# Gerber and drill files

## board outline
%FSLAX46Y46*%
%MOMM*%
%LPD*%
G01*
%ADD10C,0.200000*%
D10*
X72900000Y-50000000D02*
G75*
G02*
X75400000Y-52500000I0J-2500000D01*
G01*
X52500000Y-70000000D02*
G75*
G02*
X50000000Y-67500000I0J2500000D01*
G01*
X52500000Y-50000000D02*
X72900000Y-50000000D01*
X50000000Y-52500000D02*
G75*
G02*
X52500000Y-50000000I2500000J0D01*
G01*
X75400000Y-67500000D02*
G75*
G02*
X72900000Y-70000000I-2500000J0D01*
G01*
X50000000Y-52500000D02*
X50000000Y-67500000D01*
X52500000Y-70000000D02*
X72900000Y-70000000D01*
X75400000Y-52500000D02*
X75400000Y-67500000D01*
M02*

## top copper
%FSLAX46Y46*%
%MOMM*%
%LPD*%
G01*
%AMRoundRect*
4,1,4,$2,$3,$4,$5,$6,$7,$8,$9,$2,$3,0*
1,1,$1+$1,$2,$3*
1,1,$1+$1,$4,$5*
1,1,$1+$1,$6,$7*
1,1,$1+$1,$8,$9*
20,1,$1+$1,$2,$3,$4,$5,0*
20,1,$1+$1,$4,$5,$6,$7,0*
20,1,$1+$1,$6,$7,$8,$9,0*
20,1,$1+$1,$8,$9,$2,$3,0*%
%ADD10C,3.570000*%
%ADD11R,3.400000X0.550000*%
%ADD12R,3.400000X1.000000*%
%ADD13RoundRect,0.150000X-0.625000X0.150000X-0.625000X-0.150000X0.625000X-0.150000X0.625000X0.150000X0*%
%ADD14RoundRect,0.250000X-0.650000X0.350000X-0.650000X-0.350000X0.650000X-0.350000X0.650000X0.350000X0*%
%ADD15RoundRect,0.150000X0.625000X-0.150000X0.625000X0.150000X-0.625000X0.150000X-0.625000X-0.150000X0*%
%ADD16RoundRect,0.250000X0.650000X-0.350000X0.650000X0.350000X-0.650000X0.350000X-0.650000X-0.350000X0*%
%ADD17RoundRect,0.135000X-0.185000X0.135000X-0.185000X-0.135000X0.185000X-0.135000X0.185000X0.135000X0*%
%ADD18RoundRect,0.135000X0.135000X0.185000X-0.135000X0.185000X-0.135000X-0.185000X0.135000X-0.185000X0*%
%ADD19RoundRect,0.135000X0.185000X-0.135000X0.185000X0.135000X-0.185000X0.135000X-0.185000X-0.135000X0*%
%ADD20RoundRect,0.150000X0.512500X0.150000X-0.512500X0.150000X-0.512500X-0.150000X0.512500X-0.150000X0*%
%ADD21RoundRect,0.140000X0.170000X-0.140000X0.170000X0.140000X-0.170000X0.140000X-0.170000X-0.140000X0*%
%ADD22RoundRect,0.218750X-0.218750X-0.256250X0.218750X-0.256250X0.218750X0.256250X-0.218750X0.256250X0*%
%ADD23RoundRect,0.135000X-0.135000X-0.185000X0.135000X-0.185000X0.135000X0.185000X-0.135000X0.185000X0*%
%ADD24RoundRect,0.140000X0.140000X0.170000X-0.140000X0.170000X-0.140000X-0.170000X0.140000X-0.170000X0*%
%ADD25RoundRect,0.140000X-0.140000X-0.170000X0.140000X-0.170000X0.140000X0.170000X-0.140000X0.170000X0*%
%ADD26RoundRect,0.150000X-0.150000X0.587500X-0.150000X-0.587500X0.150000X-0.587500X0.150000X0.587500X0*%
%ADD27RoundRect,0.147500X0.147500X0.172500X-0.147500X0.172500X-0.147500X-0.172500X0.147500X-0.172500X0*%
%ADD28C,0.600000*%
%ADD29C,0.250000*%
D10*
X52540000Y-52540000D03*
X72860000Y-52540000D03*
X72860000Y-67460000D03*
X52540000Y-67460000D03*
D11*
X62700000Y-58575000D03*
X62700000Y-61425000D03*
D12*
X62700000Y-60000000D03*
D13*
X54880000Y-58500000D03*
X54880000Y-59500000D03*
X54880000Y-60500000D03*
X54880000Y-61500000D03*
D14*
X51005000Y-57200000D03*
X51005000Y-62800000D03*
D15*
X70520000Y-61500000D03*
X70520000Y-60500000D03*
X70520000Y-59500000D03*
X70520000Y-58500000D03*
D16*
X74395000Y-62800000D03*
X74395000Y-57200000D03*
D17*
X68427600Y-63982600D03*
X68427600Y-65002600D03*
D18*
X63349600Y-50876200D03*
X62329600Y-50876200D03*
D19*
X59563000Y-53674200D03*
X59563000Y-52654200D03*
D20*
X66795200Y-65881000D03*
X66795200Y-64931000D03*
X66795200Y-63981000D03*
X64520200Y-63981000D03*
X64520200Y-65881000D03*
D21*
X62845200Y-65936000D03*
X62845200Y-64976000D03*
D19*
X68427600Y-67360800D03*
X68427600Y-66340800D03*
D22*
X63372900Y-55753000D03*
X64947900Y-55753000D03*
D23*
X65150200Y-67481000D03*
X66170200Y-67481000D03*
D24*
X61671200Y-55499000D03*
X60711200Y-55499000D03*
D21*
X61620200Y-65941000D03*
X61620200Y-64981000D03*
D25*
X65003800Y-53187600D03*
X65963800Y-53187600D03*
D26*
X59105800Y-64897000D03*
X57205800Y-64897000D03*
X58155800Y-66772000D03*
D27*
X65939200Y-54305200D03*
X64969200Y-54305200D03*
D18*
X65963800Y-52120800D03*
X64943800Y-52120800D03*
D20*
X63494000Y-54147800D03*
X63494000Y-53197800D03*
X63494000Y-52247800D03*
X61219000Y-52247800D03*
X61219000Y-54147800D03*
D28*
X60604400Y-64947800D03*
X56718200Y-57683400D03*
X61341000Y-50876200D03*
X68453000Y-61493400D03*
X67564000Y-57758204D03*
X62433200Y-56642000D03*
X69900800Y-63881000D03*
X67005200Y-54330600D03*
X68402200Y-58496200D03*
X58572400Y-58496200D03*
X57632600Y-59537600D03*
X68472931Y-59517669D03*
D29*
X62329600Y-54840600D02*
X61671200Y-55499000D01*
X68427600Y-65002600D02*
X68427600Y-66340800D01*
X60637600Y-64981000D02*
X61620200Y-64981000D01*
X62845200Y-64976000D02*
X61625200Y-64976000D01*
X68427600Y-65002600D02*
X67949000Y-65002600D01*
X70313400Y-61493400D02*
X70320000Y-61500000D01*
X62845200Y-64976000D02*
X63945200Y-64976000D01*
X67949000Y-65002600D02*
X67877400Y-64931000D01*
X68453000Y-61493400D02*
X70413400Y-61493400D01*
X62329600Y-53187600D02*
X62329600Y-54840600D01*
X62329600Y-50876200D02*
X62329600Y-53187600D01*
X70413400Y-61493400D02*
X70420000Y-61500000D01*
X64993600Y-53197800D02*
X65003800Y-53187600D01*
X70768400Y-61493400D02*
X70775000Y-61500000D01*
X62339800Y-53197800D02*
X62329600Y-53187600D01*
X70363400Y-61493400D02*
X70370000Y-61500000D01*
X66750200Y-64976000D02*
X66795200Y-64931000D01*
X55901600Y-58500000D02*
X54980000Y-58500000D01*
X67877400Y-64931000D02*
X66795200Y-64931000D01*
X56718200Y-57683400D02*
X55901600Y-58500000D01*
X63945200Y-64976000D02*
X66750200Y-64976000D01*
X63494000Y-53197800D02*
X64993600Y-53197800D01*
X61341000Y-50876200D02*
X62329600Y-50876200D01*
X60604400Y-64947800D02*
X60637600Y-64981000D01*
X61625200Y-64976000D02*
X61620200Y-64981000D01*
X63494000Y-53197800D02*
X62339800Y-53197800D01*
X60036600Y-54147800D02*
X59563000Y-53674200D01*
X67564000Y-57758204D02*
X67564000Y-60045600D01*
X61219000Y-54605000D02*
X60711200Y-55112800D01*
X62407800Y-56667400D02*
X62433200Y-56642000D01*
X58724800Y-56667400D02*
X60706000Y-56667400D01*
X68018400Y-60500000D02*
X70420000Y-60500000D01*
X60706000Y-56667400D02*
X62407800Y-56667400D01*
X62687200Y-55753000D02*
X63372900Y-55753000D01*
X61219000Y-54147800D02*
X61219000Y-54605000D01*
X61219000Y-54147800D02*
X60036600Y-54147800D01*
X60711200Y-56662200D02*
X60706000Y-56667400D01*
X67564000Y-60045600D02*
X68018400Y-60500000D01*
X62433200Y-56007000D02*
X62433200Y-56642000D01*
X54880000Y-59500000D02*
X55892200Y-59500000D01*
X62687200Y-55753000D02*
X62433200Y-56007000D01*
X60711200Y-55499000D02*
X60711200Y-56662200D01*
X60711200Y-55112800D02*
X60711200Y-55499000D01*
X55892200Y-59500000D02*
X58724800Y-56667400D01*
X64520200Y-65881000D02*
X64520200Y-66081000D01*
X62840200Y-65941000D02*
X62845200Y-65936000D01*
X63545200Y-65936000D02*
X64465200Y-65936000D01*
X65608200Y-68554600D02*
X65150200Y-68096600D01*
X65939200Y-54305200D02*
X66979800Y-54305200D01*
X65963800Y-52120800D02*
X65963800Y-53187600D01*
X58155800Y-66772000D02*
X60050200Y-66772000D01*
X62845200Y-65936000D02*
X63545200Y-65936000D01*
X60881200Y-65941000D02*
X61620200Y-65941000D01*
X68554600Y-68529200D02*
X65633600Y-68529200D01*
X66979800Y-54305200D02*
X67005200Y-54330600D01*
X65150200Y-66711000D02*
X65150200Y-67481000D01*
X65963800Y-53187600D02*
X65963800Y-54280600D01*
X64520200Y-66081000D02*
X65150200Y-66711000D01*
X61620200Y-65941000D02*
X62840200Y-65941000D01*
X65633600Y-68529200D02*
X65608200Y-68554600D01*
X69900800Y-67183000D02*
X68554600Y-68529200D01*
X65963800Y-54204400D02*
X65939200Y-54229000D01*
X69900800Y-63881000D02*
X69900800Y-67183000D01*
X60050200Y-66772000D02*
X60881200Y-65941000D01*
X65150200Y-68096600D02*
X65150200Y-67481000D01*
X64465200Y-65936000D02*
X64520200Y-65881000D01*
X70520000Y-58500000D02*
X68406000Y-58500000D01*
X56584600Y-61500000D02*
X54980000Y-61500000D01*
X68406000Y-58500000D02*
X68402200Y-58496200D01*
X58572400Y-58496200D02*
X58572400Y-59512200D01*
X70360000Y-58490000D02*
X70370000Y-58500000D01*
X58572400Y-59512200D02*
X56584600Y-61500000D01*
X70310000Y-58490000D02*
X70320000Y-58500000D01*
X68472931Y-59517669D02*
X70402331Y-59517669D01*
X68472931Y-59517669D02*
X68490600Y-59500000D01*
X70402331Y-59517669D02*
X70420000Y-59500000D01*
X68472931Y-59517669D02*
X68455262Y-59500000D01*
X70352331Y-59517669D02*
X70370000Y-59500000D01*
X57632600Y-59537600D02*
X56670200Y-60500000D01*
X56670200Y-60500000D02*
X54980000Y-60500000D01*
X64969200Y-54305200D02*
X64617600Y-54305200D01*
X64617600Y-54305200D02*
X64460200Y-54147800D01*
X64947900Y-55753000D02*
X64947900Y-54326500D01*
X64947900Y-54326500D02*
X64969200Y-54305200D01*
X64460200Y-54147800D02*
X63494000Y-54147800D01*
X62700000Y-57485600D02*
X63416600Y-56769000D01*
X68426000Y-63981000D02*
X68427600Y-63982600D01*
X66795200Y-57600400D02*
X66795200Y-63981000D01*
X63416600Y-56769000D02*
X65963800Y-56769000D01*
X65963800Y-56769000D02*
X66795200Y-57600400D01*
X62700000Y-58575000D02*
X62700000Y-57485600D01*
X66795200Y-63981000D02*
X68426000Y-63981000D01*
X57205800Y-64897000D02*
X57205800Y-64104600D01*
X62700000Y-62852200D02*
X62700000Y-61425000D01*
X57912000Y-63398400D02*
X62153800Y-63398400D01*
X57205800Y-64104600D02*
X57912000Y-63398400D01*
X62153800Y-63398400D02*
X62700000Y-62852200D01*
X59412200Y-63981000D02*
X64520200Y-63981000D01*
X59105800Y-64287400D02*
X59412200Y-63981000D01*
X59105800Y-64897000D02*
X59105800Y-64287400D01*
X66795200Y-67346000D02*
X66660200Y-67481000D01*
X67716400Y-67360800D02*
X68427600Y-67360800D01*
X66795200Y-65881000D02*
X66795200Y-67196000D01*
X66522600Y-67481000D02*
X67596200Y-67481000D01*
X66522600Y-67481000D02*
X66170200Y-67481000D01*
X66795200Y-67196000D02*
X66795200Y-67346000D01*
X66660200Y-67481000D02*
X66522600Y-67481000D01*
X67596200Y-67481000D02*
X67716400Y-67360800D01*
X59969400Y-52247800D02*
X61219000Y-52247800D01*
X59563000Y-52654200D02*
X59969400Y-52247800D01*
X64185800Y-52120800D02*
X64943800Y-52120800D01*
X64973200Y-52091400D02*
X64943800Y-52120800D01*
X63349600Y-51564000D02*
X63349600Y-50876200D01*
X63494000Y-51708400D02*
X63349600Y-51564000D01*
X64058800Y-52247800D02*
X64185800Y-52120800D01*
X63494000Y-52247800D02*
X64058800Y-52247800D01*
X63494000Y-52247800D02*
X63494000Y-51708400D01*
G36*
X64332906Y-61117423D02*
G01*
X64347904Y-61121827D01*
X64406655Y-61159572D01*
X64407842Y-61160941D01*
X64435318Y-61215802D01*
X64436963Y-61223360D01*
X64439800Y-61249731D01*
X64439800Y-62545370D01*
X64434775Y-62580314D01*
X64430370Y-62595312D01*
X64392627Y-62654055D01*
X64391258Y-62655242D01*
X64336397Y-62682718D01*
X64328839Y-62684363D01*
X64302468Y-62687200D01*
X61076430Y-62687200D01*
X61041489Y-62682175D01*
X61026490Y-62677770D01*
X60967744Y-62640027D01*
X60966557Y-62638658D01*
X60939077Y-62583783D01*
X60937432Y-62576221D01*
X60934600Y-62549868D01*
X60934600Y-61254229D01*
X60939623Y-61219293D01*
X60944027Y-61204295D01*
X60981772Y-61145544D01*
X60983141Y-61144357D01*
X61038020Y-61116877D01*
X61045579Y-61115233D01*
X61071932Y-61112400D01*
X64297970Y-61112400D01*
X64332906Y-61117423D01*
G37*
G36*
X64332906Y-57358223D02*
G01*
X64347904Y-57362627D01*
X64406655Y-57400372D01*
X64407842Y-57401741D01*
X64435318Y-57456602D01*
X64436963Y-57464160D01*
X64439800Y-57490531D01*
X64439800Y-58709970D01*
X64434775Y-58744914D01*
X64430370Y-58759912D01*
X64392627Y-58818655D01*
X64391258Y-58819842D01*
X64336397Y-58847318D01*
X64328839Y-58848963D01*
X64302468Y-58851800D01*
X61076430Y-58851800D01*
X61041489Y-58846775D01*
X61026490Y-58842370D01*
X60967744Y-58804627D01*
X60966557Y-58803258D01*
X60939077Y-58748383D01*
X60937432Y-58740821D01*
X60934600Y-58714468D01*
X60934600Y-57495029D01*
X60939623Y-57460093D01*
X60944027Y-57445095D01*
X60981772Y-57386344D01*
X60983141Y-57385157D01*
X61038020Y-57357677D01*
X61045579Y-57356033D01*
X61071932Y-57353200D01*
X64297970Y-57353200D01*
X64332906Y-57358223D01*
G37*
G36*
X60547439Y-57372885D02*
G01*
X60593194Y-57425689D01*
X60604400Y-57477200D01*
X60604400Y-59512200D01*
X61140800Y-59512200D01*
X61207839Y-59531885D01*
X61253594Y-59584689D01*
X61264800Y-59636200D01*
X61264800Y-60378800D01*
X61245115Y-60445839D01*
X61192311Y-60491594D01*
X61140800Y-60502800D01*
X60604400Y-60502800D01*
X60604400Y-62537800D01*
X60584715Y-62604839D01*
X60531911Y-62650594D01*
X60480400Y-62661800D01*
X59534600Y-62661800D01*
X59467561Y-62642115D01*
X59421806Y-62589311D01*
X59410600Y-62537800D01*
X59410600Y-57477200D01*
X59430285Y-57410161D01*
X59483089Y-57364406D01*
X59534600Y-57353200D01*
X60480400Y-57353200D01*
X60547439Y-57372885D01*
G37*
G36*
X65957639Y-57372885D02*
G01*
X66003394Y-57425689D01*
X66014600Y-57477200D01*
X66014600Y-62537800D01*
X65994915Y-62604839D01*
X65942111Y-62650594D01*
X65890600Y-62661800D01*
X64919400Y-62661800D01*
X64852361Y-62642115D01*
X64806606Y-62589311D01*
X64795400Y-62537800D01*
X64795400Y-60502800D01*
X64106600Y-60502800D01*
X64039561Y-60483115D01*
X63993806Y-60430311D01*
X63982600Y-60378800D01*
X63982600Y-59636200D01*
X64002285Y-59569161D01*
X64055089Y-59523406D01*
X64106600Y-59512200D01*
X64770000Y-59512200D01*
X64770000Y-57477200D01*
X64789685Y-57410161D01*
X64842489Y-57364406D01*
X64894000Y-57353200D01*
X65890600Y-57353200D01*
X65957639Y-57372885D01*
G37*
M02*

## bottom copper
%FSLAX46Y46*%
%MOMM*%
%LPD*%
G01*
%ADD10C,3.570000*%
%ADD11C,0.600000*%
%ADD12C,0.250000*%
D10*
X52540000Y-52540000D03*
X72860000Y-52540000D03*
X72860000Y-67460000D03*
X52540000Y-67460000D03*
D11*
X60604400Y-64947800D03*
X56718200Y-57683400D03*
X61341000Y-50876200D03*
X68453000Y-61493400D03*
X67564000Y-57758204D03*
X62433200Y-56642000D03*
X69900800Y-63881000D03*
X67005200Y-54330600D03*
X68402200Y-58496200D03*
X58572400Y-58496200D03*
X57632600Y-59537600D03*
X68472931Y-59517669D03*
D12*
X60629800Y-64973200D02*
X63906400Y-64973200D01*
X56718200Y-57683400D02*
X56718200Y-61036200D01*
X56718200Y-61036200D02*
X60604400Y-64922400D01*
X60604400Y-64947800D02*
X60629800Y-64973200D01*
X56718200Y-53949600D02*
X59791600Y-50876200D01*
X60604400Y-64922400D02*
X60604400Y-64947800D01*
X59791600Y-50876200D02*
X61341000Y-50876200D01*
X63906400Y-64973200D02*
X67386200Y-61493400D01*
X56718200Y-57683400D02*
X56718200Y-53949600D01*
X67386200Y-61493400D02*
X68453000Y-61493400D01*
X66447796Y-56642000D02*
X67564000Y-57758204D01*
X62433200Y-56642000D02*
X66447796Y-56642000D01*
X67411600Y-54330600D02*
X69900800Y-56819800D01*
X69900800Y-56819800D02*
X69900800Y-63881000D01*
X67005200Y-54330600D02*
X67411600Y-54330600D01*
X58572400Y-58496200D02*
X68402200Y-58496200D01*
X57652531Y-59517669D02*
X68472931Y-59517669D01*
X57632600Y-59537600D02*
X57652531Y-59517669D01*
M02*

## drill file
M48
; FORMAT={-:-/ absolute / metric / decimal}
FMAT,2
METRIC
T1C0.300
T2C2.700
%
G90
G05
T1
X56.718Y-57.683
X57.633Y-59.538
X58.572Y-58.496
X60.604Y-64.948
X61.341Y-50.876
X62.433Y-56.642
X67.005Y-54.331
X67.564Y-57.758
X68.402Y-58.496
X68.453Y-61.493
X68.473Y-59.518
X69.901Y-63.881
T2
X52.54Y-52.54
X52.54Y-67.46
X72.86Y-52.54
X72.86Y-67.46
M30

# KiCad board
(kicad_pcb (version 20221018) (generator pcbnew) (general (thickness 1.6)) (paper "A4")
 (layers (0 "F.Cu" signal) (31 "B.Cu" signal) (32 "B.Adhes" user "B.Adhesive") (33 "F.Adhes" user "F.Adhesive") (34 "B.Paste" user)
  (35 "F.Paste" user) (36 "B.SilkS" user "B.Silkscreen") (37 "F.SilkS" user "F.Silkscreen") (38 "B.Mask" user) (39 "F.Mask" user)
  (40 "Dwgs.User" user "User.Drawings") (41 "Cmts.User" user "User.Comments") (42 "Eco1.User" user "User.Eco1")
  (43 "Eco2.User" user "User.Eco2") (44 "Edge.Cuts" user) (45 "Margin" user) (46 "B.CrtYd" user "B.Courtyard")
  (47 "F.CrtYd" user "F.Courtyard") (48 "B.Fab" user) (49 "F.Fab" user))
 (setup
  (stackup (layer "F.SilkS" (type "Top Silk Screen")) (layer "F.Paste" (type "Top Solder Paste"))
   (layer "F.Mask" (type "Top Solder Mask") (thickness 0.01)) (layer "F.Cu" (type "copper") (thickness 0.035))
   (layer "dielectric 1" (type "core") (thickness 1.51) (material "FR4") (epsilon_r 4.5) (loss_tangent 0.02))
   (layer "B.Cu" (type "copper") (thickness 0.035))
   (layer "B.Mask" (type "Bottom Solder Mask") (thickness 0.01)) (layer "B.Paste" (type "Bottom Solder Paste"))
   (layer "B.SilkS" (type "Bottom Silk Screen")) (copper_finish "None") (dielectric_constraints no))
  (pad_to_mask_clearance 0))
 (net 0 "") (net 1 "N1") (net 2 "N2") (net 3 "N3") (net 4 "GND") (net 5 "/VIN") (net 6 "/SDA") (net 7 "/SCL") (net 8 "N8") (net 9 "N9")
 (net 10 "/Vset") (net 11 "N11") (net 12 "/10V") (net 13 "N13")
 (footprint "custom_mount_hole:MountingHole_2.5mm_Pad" (layer "F.Cu") (at 52.54 52.54)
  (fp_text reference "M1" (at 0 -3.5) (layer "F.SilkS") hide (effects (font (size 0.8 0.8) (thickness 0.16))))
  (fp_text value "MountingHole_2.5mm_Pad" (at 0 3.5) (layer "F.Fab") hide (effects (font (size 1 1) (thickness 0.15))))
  (pad "~" thru_hole circle (at 0 0) (size 3.57 3.57) (drill 2.7) (layers "*.Cu" "*.Mask")))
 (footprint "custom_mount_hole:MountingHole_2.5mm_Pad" (layer "F.Cu") (at 72.86 52.54)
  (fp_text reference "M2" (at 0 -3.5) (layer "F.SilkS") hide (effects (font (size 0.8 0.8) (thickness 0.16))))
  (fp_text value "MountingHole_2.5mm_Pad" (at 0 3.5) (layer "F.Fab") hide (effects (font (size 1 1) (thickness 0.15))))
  (pad "~" thru_hole circle (at 0 0) (size 3.57 3.57) (drill 2.7) (layers "*.Cu" "*.Mask")))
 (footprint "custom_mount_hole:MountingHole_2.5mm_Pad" (layer "F.Cu") (at 72.86 67.46)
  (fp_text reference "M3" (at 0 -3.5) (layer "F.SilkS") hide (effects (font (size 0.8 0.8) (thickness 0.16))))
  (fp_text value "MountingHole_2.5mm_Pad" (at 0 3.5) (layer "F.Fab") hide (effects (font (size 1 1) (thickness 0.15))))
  (pad "~" thru_hole circle (at 0 0) (size 3.57 3.57) (drill 2.7) (layers "*.Cu" "*.Mask")))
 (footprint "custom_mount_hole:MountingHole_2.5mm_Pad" (layer "F.Cu") (at 52.54 67.46)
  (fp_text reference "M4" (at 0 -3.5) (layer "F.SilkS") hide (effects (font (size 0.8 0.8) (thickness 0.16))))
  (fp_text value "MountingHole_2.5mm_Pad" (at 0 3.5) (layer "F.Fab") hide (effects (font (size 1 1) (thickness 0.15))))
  (pad "~" thru_hole circle (at 0 0) (size 3.57 3.57) (drill 2.7) (layers "*.Cu" "*.Mask")))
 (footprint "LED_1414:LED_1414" (layer "F.Cu") (at 62.7 60 -90)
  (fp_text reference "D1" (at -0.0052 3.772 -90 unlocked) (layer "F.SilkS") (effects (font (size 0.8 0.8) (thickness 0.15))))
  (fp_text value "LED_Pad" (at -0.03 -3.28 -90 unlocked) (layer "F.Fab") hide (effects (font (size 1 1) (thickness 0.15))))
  (pad "1" smd rect (at -1.425 0 270) (size 0.55 3.4) (layers "F.Cu" "F.Paste" "F.Mask") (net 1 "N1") (thermal_bridge_angle 45))
  (pad "2" smd rect (at 1.425 0 270) (size 0.55 3.4) (layers "F.Cu" "F.Paste" "F.Mask") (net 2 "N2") (thermal_bridge_angle 45))
  (pad "3" smd rect (at 0 0 270) (size 1 3.4) (layers "F.Cu" "F.Paste" "F.Mask") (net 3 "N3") (thermal_bridge_angle 45)))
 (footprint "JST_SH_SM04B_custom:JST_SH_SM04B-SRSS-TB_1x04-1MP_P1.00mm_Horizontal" (layer "F.Cu") (at 52.88 60 -90)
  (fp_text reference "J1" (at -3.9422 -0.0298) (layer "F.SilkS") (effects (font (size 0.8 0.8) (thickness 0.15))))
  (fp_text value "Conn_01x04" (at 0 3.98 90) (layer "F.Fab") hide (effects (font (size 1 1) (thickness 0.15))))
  (pad "1" smd roundrect (at -1.5 -2 270) (size 0.6 1.55) (layers "F.Cu" "F.Paste" "F.Mask") (roundrect_rratio 0.25) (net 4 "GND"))
  (pad "2" smd roundrect (at -0.5 -2 270) (size 0.6 1.55) (layers "F.Cu" "F.Paste" "F.Mask") (roundrect_rratio 0.25) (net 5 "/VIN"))
  (pad "3" smd roundrect (at 0.5 -2 270) (size 0.6 1.55) (layers "F.Cu" "F.Paste" "F.Mask") (roundrect_rratio 0.25) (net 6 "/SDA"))
  (pad "4" smd roundrect (at 1.5 -2 270) (size 0.6 1.55) (layers "F.Cu" "F.Paste" "F.Mask") (roundrect_rratio 0.25) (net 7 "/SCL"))
  (pad "MP" smd roundrect (at -2.8 1.875 270) (size 1.2 1.8) (layers "F.Cu" "F.Paste" "F.Mask") (roundrect_rratio 0.2083333333))
  (pad "MP" smd roundrect (at 2.8 1.875 270) (size 1.2 1.8) (layers "F.Cu" "F.Paste" "F.Mask") (roundrect_rratio 0.2083333333)))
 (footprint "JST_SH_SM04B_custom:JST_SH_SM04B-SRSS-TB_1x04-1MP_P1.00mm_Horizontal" (layer "F.Cu") (at 72.52 60 90)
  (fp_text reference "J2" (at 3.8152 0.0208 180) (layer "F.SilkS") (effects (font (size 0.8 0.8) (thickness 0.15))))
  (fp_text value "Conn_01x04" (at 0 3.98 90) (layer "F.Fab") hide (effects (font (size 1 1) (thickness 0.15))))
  (pad "1" smd roundrect (at -1.5 -2 90) (size 0.6 1.55) (layers "F.Cu" "F.Paste" "F.Mask") (roundrect_rratio 0.25) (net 4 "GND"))
  (pad "2" smd roundrect (at -0.5 -2 90) (size 0.6 1.55) (layers "F.Cu" "F.Paste" "F.Mask") (roundrect_rratio 0.25) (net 5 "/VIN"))
  (pad "3" smd roundrect (at 0.5 -2 90) (size 0.6 1.55) (layers "F.Cu" "F.Paste" "F.Mask") (roundrect_rratio 0.25) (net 6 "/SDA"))
  (pad "4" smd roundrect (at 1.5 -2 90) (size 0.6 1.55) (layers "F.Cu" "F.Paste" "F.Mask") (roundrect_rratio 0.25) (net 7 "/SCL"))
  (pad "MP" smd roundrect (at -2.8 1.875 90) (size 1.2 1.8) (layers "F.Cu" "F.Paste" "F.Mask") (roundrect_rratio 0.2083333333))
  (pad "MP" smd roundrect (at 2.8 1.875 90) (size 1.2 1.8) (layers "F.Cu" "F.Paste" "F.Mask") (roundrect_rratio 0.2083333333)))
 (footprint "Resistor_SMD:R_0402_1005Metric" (layer "F.Cu") (at 68.4276 64.4926 -90)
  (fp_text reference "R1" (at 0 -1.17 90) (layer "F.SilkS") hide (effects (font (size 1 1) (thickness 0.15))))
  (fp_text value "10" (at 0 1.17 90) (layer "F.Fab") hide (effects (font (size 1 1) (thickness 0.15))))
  (pad "1" smd roundrect (at -0.51 0 270) (size 0.54 0.64) (layers "F.Cu" "F.Paste" "F.Mask") (roundrect_rratio 0.25) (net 1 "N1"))
  (pad "2" smd roundrect (at 0.51 0 270) (size 0.54 0.64) (layers "F.Cu" "F.Paste" "F.Mask") (roundrect_rratio 0.25) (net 4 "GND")))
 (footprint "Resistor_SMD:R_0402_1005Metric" (layer "F.Cu") (at 62.8396 50.8762 180)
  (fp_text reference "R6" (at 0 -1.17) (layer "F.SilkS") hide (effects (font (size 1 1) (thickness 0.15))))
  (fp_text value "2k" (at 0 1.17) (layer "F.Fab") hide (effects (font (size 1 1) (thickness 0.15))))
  (pad "1" smd roundrect (at -0.51 0 180) (size 0.54 0.64) (layers "F.Cu" "F.Paste" "F.Mask") (roundrect_rratio 0.25) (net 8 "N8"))
  (pad "2" smd roundrect (at 0.51 0 180) (size 0.54 0.64) (layers "F.Cu" "F.Paste" "F.Mask") (roundrect_rratio 0.25) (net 4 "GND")))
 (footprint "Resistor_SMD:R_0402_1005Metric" (layer "F.Cu") (at 59.563 53.1642 90)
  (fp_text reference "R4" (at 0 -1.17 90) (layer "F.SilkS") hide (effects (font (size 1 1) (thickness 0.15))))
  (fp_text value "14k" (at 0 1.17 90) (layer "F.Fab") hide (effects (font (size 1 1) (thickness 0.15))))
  (pad "1" smd roundrect (at -0.51 0 90) (size 0.54 0.64) (layers "F.Cu" "F.Paste" "F.Mask") (roundrect_rratio 0.25) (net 5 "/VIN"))
  (pad "2" smd roundrect (at 0.51 0 90) (size 0.54 0.64) (layers "F.Cu" "F.Paste" "F.Mask") (roundrect_rratio 0.25) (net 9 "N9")))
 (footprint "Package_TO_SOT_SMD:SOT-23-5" (layer "F.Cu") (at 65.6577 64.931 180)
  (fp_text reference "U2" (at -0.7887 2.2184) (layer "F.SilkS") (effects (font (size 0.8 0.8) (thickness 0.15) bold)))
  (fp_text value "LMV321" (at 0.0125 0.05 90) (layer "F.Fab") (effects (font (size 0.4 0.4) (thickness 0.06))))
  (pad "1" smd roundrect (at -1.1375 -0.95 180) (size 1.325 0.6) (layers "F.Cu" "F.Paste" "F.Mask") (roundrect_rratio 0.25) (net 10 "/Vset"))
  (pad "2" smd roundrect (at -1.1375 0 180) (size 1.325 0.6) (layers "F.Cu" "F.Paste" "F.Mask") (roundrect_rratio 0.25) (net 4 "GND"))
  (pad "3" smd roundrect (at -1.1375 0.95 180) (size 1.325 0.6) (layers "F.Cu" "F.Paste" "F.Mask") (roundrect_rratio 0.25) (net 1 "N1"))
  (pad "4" smd roundrect (at 1.1375 0.95 180) (size 1.325 0.6) (layers "F.Cu" "F.Paste" "F.Mask") (roundrect_rratio 0.25) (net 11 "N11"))
  (pad "5" smd roundrect (at 1.1375 -0.95 180) (size 1.325 0.6) (layers "F.Cu" "F.Paste" "F.Mask") (roundrect_rratio 0.25) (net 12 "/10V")))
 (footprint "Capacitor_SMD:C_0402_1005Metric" (layer "F.Cu") (at 62.8452 65.456 90)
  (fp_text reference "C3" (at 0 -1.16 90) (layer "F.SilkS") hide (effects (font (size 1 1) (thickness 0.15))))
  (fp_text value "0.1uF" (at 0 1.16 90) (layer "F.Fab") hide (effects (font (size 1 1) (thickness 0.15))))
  (pad "1" smd roundrect (at -0.48 0 90) (size 0.56 0.62) (layers "F.Cu" "F.Paste" "F.Mask") (roundrect_rratio 0.25) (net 12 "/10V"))
  (pad "2" smd roundrect (at 0.48 0 90) (size 0.56 0.62) (layers "F.Cu" "F.Paste" "F.Mask") (roundrect_rratio 0.25) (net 4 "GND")))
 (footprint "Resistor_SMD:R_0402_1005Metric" (layer "F.Cu") (at 68.4276 66.8508 90)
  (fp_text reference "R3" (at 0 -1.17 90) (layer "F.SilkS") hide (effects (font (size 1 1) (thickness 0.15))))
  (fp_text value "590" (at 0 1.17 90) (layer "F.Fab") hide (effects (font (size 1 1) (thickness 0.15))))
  (pad "1" smd roundrect (at -0.51 0 90) (size 0.54 0.64) (layers "F.Cu" "F.Paste" "F.Mask") (roundrect_rratio 0.25) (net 10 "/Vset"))
  (pad "2" smd roundrect (at 0.51 0 90) (size 0.54 0.64) (layers "F.Cu" "F.Paste" "F.Mask") (roundrect_rratio 0.25) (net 4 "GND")))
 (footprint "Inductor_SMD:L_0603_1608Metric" (layer "F.Cu") (at 64.1604 55.753)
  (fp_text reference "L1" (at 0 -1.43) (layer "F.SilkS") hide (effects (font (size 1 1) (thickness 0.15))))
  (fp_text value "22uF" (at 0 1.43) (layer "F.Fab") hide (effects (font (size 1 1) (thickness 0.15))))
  (pad "1" smd roundrect (at -0.7875 0) (size 0.875 0.95) (layers "F.Cu" "F.Paste" "F.Mask") (roundrect_rratio 0.25) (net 5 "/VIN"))
  (pad "2" smd roundrect (at 0.7875 0) (size 0.875 0.95) (layers "F.Cu" "F.Paste" "F.Mask") (roundrect_rratio 0.25) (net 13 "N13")))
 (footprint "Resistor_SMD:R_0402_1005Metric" (layer "F.Cu") (at 65.6602 67.481)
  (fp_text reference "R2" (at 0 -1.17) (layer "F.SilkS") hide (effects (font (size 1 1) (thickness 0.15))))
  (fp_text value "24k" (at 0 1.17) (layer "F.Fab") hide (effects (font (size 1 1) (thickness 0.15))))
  (pad "1" smd roundrect (at -0.51 0) (size 0.54 0.64) (layers "F.Cu" "F.Paste" "F.Mask") (roundrect_rratio 0.25) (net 12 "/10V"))
  (pad "2" smd roundrect (at 0.51 0) (size 0.54 0.64) (layers "F.Cu" "F.Paste" "F.Mask") (roundrect_rratio 0.25) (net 10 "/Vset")))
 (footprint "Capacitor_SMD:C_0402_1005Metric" (layer "F.Cu") (at 61.1912 55.499 180)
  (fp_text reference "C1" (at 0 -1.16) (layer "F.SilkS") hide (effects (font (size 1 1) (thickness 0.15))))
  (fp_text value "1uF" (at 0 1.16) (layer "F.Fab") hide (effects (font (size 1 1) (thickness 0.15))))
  (pad "1" smd roundrect (at -0.48 0 180) (size 0.56 0.62) (layers "F.Cu" "F.Paste" "F.Mask") (roundrect_rratio 0.25) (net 4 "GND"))
  (pad "2" smd roundrect (at 0.48 0 180) (size 0.56 0.62) (layers "F.Cu" "F.Paste" "F.Mask") (roundrect_rratio 0.25) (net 5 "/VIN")))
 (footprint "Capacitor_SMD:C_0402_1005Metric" (layer "F.Cu") (at 61.6202 65.461 90)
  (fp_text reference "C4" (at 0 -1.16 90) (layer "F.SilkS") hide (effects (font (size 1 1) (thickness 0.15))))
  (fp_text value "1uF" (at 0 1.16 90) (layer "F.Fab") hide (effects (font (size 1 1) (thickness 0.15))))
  (pad "1" smd roundrect (at -0.48 0 90) (size 0.56 0.62) (layers "F.Cu" "F.Paste" "F.Mask") (roundrect_rratio 0.25) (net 12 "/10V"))
  (pad "2" smd roundrect (at 0.48 0 90) (size 0.56 0.62) (layers "F.Cu" "F.Paste" "F.Mask") (roundrect_rratio 0.25) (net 4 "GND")))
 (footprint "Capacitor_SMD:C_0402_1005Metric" (layer "F.Cu") (at 65.4838 53.1876)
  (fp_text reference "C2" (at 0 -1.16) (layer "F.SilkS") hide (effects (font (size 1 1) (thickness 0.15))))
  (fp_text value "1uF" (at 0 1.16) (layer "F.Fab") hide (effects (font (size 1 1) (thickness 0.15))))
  (pad "1" smd roundrect (at -0.48 0) (size 0.56 0.62) (layers "F.Cu" "F.Paste" "F.Mask") (roundrect_rratio 0.25) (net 4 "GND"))
  (pad "2" smd roundrect (at 0.48 0) (size 0.56 0.62) (layers "F.Cu" "F.Paste" "F.Mask") (roundrect_rratio 0.25) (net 12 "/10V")))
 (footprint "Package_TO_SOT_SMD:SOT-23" (layer "F.Cu") (at 58.1558 65.8345 -90)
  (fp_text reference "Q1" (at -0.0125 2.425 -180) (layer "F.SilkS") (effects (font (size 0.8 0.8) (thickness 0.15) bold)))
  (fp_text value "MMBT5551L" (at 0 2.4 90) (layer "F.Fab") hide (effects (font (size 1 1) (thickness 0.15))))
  (pad "1" smd roundrect (at -0.9375 -0.95 270) (size 1.475 0.6) (layers "F.Cu" "F.Paste" "F.Mask") (roundrect_rratio 0.25) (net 11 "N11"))
  (pad "2" smd roundrect (at -0.9375 0.95 270) (size 1.475 0.6) (layers "F.Cu" "F.Paste" "F.Mask") (roundrect_rratio 0.25) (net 2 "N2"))
  (pad "3" smd roundrect (at 0.9375 0 270) (size 1.475 0.6) (layers "F.Cu" "F.Paste" "F.Mask") (roundrect_rratio 0.25) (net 12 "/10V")))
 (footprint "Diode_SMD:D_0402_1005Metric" (layer "F.Cu") (at 65.4542 54.3052 180)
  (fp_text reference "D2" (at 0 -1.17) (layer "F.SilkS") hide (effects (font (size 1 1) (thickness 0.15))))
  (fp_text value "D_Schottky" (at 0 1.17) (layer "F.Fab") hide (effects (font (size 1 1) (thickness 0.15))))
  (pad "1" smd roundrect (at -0.485 0 180) (size 0.59 0.64) (layers "F.Cu" "F.Paste" "F.Mask") (roundrect_rratio 0.25) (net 12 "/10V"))
  (pad "2" smd roundrect (at 0.485 0 180) (size 0.59 0.64) (layers "F.Cu" "F.Paste" "F.Mask") (roundrect_rratio 0.25) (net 13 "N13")))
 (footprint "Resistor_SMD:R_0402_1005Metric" (layer "F.Cu") (at 65.4538 52.1208 180)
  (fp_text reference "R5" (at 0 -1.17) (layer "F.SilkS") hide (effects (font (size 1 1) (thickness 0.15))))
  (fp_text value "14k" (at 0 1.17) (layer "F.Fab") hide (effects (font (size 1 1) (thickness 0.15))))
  (pad "1" smd roundrect (at -0.51 0 180) (size 0.54 0.64) (layers "F.Cu" "F.Paste" "F.Mask") (roundrect_rratio 0.25) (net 12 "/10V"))
  (pad "2" smd roundrect (at 0.51 0 180) (size 0.54 0.64) (layers "F.Cu" "F.Paste" "F.Mask") (roundrect_rratio 0.25) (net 8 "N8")))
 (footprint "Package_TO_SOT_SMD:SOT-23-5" (layer "F.Cu") (at 62.3565 53.1978 180)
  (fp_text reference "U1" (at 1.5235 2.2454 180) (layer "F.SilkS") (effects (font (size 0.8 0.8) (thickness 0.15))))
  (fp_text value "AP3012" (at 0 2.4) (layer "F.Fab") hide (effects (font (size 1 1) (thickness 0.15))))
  (pad "1" smd roundrect (at -1.1375 -0.95 180) (size 1.325 0.6) (layers "F.Cu" "F.Paste" "F.Mask") (roundrect_rratio 0.25) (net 13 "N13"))
  (pad "2" smd roundrect (at -1.1375 0 180) (size 1.325 0.6) (layers "F.Cu" "F.Paste" "F.Mask") (roundrect_rratio 0.25) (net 4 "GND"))
  (pad "3" smd roundrect (at -1.1375 0.95 180) (size 1.325 0.6) (layers "F.Cu" "F.Paste" "F.Mask") (roundrect_rratio 0.25) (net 8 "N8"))
  (pad "4" smd roundrect (at 1.1375 0.95 180) (size 1.325 0.6) (layers "F.Cu" "F.Paste" "F.Mask") (roundrect_rratio 0.25) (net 9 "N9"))
  (pad "5" smd roundrect (at 1.1375 -0.95 180) (size 1.325 0.6) (layers "F.Cu" "F.Paste" "F.Mask") (roundrect_rratio 0.25) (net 5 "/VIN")))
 (gr_arc (start 72.9 50) (mid 74.667767 50.732233) (end 75.4 52.5) (stroke (width 0.2) (type solid)) (layer "Edge.Cuts"))
 (gr_arc (start 52.5 70) (mid 50.732233 69.267767) (end 50 67.5) (stroke (width 0.2) (type solid)) (layer "Edge.Cuts"))
 (gr_line (start 52.5 50) (end 72.9 50) (stroke (width 0.2) (type solid)) (layer "Edge.Cuts"))
 (gr_arc (start 50 52.5) (mid 50.732233 50.732233) (end 52.5 50) (stroke (width 0.2) (type solid)) (layer "Edge.Cuts"))
 (gr_arc (start 75.4 67.5) (mid 74.667767 69.267767) (end 72.9 70) (stroke (width 0.2) (type solid)) (layer "Edge.Cuts"))
 (gr_line (start 50 52.5) (end 50 67.5) (stroke (width 0.2) (type solid)) (layer "Edge.Cuts"))
 (gr_line (start 52.5 70) (end 72.9 70) (stroke (width 0.2) (type solid)) (layer "Edge.Cuts"))
 (gr_line (start 75.4 52.5) (end 75.4 67.5) (stroke (width 0.2) (type solid)) (layer "Edge.Cuts"))
 (segment (start 62.3296 54.8406) (end 61.6712 55.499) (width 0.25) (layer "F.Cu") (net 4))
 (segment (start 68.4276 65.0026) (end 68.4276 66.3408) (width 0.25) (layer "F.Cu") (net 4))
 (segment (start 60.6376 64.981) (end 61.6202 64.981) (width 0.25) (layer "F.Cu") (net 4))
 (segment (start 62.8452 64.976) (end 61.6252 64.976) (width 0.25) (layer "F.Cu") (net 4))
 (segment (start 68.4276 65.0026) (end 67.949 65.0026) (width 0.25) (layer "F.Cu") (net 4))
 (segment (start 70.3134 61.4934) (end 70.32 61.5) (width 0.25) (layer "F.Cu") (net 4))
 (segment (start 62.8452 64.976) (end 63.9452 64.976) (width 0.25) (layer "F.Cu") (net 4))
 (segment (start 67.949 65.0026) (end 67.8774 64.931) (width 0.25) (layer "F.Cu") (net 4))
 (segment (start 68.453 61.4934) (end 70.4134 61.4934) (width 0.25) (layer "F.Cu") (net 4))
 (segment (start 62.3296 53.1876) (end 62.3296 54.8406) (width 0.25) (layer "F.Cu") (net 4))
 (segment (start 62.3296 50.8762) (end 62.3296 53.1876) (width 0.25) (layer "F.Cu") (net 4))
 (segment (start 70.4134 61.4934) (end 70.42 61.5) (width 0.25) (layer "F.Cu") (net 4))
 (segment (start 64.9936 53.1978) (end 65.0038 53.1876) (width 0.25) (layer "F.Cu") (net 4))
 (segment (start 70.7684 61.4934) (end 70.775 61.5) (width 0.25) (layer "F.Cu") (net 4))
 (segment (start 62.3398 53.1978) (end 62.3296 53.1876) (width 0.25) (layer "F.Cu") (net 4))
 (segment (start 70.3634 61.4934) (end 70.37 61.5) (width 0.25) (layer "F.Cu") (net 4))
 (segment (start 66.7502 64.976) (end 66.7952 64.931) (width 0.25) (layer "F.Cu") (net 4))
 (segment (start 55.9016 58.5) (end 54.98 58.5) (width 0.25) (layer "F.Cu") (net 4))
 (segment (start 67.8774 64.931) (end 66.7952 64.931) (width 0.25) (layer "F.Cu") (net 4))
 (segment (start 56.7182 57.6834) (end 55.9016 58.5) (width 0.25) (layer "F.Cu") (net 4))
 (segment (start 63.9452 64.976) (end 66.7502 64.976) (width 0.25) (layer "F.Cu") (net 4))
 (segment (start 63.494 53.1978) (end 64.9936 53.1978) (width 0.25) (layer "F.Cu") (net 4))
 (segment (start 61.341 50.8762) (end 62.3296 50.8762) (width 0.25) (layer "F.Cu") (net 4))
 (segment (start 60.6044 64.9478) (end 60.6376 64.981) (width 0.25) (layer "F.Cu") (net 4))
 (segment (start 61.6252 64.976) (end 61.6202 64.981) (width 0.25) (layer "F.Cu") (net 4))
 (segment (start 63.494 53.1978) (end 62.3398 53.1978) (width 0.25) (layer "F.Cu") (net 4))
 (via (at 60.6044 64.9478) (size 0.6) (drill 0.3) (layers "F.Cu" "B.Cu") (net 4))
 (via (at 56.7182 57.6834) (size 0.6) (drill 0.3) (layers "F.Cu" "B.Cu") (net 4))
 (via (at 61.341 50.8762) (size 0.6) (drill 0.3) (layers "F.Cu" "B.Cu") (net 4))
 (via (at 68.453 61.4934) (size 0.6) (drill 0.3) (layers "F.Cu" "B.Cu") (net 4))
 (segment (start 60.6298 64.9732) (end 63.9064 64.9732) (width 0.25) (layer "B.Cu") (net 4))
 (segment (start 56.7182 57.6834) (end 56.7182 61.0362) (width 0.25) (layer "B.Cu") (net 4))
 (segment (start 56.7182 61.0362) (end 60.6044 64.9224) (width 0.25) (layer "B.Cu") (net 4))
 (segment (start 60.6044 64.9478) (end 60.6298 64.9732) (width 0.25) (layer "B.Cu") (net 4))
 (segment (start 56.7182 53.9496) (end 59.7916 50.8762) (width 0.25) (layer "B.Cu") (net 4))
 (segment (start 60.6044 64.9224) (end 60.6044 64.9478) (width 0.25) (layer "B.Cu") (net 4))
 (segment (start 59.7916 50.8762) (end 61.341 50.8762) (width 0.25) (layer "B.Cu") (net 4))
 (segment (start 63.9064 64.9732) (end 67.3862 61.4934) (width 0.25) (layer "B.Cu") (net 4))
 (segment (start 56.7182 57.6834) (end 56.7182 53.9496) (width 0.25) (layer "B.Cu") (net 4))
 (segment (start 67.3862 61.4934) (end 68.453 61.4934) (width 0.25) (layer "B.Cu") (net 4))
 (segment (start 60.0366 54.1478) (end 59.563 53.6742) (width 0.25) (layer "F.Cu") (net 5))
 (segment (start 67.564 57.758204) (end 67.564 60.0456) (width 0.25) (layer "F.Cu") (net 5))
 (segment (start 61.219 54.605) (end 60.7112 55.1128) (width 0.25) (layer "F.Cu") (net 5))
 (segment (start 62.4078 56.6674) (end 62.4332 56.642) (width 0.25) (layer "F.Cu") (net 5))
 (segment (start 58.7248 56.6674) (end 60.706 56.6674) (width 0.25) (layer "F.Cu") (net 5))
 (segment (start 68.0184 60.5) (end 70.42 60.5) (width 0.25) (layer "F.Cu") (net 5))
 (segment (start 60.706 56.6674) (end 62.4078 56.6674) (width 0.25) (layer "F.Cu") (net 5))
 (segment (start 62.6872 55.753) (end 63.3729 55.753) (width 0.25) (layer "F.Cu") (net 5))
 (segment (start 61.219 54.1478) (end 61.219 54.605) (width 0.25) (layer "F.Cu") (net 5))
 (segment (start 61.219 54.1478) (end 60.0366 54.1478) (width 0.25) (layer "F.Cu") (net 5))
 (segment (start 60.7112 56.6622) (end 60.706 56.6674) (width 0.25) (layer "F.Cu") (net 5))
 (segment (start 67.564 60.0456) (end 68.0184 60.5) (width 0.25) (layer "F.Cu") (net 5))
 (segment (start 62.4332 56.007) (end 62.4332 56.642) (width 0.25) (layer "F.Cu") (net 5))
 (segment (start 54.88 59.5) (end 55.8922 59.5) (width 0.25) (layer "F.Cu") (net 5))
 (segment (start 62.6872 55.753) (end 62.4332 56.007) (width 0.25) (layer "F.Cu") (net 5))
 (segment (start 60.7112 55.499) (end 60.7112 56.6622) (width 0.25) (layer "F.Cu") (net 5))
 (segment (start 60.7112 55.1128) (end 60.7112 55.499) (width 0.25) (layer "F.Cu") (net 5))
 (segment (start 55.8922 59.5) (end 58.7248 56.6674) (width 0.25) (layer "F.Cu") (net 5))
 (via (at 67.564 57.758204) (size 0.6) (drill 0.3) (layers "F.Cu" "B.Cu") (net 5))
 (via (at 62.4332 56.642) (size 0.6) (drill 0.3) (layers "F.Cu" "B.Cu") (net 5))
 (segment (start 66.447796 56.642) (end 67.564 57.758204) (width 0.25) (layer "B.Cu") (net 5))
 (segment (start 62.4332 56.642) (end 66.447796 56.642) (width 0.25) (layer "B.Cu") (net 5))
 (segment (start 64.5202 65.881) (end 64.5202 66.081) (width 0.25) (layer "F.Cu") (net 12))
 (segment (start 62.8402 65.941) (end 62.8452 65.936) (width 0.25) (layer "F.Cu") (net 12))
 (segment (start 63.5452 65.936) (end 64.4652 65.936) (width 0.25) (layer "F.Cu") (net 12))
 (segment (start 65.6082 68.5546) (end 65.1502 68.0966) (width 0.25) (layer "F.Cu") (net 12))
 (segment (start 65.9392 54.3052) (end 66.9798 54.3052) (width 0.25) (layer "F.Cu") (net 12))
 (segment (start 65.9638 52.1208) (end 65.9638 53.1876) (width 0.25) (layer "F.Cu") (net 12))
 (segment (start 58.1558 66.772) (end 60.0502 66.772) (width 0.25) (layer "F.Cu") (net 12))
 (segment (start 62.8452 65.936) (end 63.5452 65.936) (width 0.25) (layer "F.Cu") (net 12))
 (segment (start 60.8812 65.941) (end 61.6202 65.941) (width 0.25) (layer "F.Cu") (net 12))
 (segment (start 68.5546 68.5292) (end 65.6336 68.5292) (width 0.25) (layer "F.Cu") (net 12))
 (segment (start 66.9798 54.3052) (end 67.0052 54.3306) (width 0.25) (layer "F.Cu") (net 12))
 (segment (start 65.1502 66.711) (end 65.1502 67.481) (width 0.25) (layer "F.Cu") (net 12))
 (segment (start 65.9638 53.1876) (end 65.9638 54.2806) (width 0.25) (layer "F.Cu") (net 12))
 (segment (start 64.5202 66.081) (end 65.1502 66.711) (width 0.25) (layer "F.Cu") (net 12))
 (segment (start 61.6202 65.941) (end 62.8402 65.941) (width 0.25) (layer "F.Cu") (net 12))
 (segment (start 65.6336 68.5292) (end 65.6082 68.5546) (width 0.25) (layer "F.Cu") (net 12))
 (segment (start 69.9008 67.183) (end 68.5546 68.5292) (width 0.25) (layer "F.Cu") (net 12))
 (segment (start 65.9638 54.2044) (end 65.9392 54.229) (width 0.25) (layer "F.Cu") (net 12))
 (segment (start 69.9008 63.881) (end 69.9008 67.183) (width 0.25) (layer "F.Cu") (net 12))
 (segment (start 60.0502 66.772) (end 60.8812 65.941) (width 0.25) (layer "F.Cu") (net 12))
 (segment (start 65.1502 68.0966) (end 65.1502 67.481) (width 0.25) (layer "F.Cu") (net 12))
 (segment (start 64.4652 65.936) (end 64.5202 65.881) (width 0.25) (layer "F.Cu") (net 12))
 (via (at 69.9008 63.881) (size 0.6) (drill 0.3) (layers "F.Cu" "B.Cu") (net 12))
 (via (at 67.0052 54.3306) (size 0.6) (drill 0.3) (layers "F.Cu" "B.Cu") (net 12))
 (segment (start 67.4116 54.3306) (end 69.9008 56.8198) (width 0.25) (layer "B.Cu") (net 12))
 (segment (start 69.9008 56.8198) (end 69.9008 63.881) (width 0.25) (layer "B.Cu") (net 12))
 (segment (start 67.0052 54.3306) (end 67.4116 54.3306) (width 0.25) (layer "B.Cu") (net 12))
 (segment (start 70.52 58.5) (end 68.406 58.5) (width 0.25) (layer "F.Cu") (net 7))
 (segment (start 56.5846 61.5) (end 54.98 61.5) (width 0.25) (layer "F.Cu") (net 7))
 (segment (start 68.406 58.5) (end 68.4022 58.4962) (width 0.25) (layer "F.Cu") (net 7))
 (segment (start 58.5724 58.4962) (end 58.5724 59.5122) (width 0.25) (layer "F.Cu") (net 7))
 (segment (start 70.36 58.49) (end 70.37 58.5) (width 0.25) (layer "F.Cu") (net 7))
 (segment (start 58.5724 59.5122) (end 56.5846 61.5) (width 0.25) (layer "F.Cu") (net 7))
 (segment (start 70.31 58.49) (end 70.32 58.5) (width 0.25) (layer "F.Cu") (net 7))
 (via (at 68.4022 58.4962) (size 0.6) (drill 0.3) (layers "F.Cu" "B.Cu") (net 7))
 (via (at 58.5724 58.4962) (size 0.6) (drill 0.3) (layers "F.Cu" "B.Cu") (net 7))
 (segment (start 58.5724 58.4962) (end 68.4022 58.4962) (width 0.25) (layer "B.Cu") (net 7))
 (segment (start 68.472931 59.517669) (end 70.402331 59.517669) (width 0.25) (layer "F.Cu") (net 6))
 (segment (start 68.472931 59.517669) (end 68.4906 59.5) (width 0.25) (layer "F.Cu") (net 6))
 (segment (start 70.402331 59.517669) (end 70.42 59.5) (width 0.25) (layer "F.Cu") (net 6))
 (segment (start 68.472931 59.517669) (end 68.455262 59.5) (width 0.25) (layer "F.Cu") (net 6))
 (segment (start 70.352331 59.517669) (end 70.37 59.5) (width 0.25) (layer "F.Cu") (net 6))
 (segment (start 57.6326 59.5376) (end 56.6702 60.5) (width 0.25) (layer "F.Cu") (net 6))
 (segment (start 56.6702 60.5) (end 54.98 60.5) (width 0.25) (layer "F.Cu") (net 6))
 (via (at 57.6326 59.5376) (size 0.6) (drill 0.3) (layers "F.Cu" "B.Cu") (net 6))
 (via (at 68.472931 59.517669) (size 0.6) (drill 0.3) (layers "F.Cu" "B.Cu") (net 6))
 (segment (start 57.652531 59.517669) (end 68.472931 59.517669) (width 0.25) (layer "B.Cu") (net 6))
 (segment (start 57.6326 59.5376) (end 57.652531 59.517669) (width 0.25) (layer "B.Cu") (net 6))
 (segment (start 64.9692 54.3052) (end 64.6176 54.3052) (width 0.25) (layer "F.Cu") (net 13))
 (segment (start 64.6176 54.3052) (end 64.4602 54.1478) (width 0.25) (layer "F.Cu") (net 13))
 (segment (start 64.9479 55.753) (end 64.9479 54.3265) (width 0.25) (layer "F.Cu") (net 13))
 (segment (start 64.9479 54.3265) (end 64.9692 54.3052) (width 0.25) (layer "F.Cu") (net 13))
 (segment (start 64.4602 54.1478) (end 63.494 54.1478) (width 0.25) (layer "F.Cu") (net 13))
 (segment (start 62.7 57.4856) (end 63.4166 56.769) (width 0.25) (layer "F.Cu") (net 1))
 (segment (start 68.426 63.981) (end 68.4276 63.9826) (width 0.25) (layer "F.Cu") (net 1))
 (segment (start 66.7952 57.6004) (end 66.7952 63.981) (width 0.25) (layer "F.Cu") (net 1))
 (segment (start 63.4166 56.769) (end 65.9638 56.769) (width 0.25) (layer "F.Cu") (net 1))
 (segment (start 65.9638 56.769) (end 66.7952 57.6004) (width 0.25) (layer "F.Cu") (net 1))
 (segment (start 62.7 58.575) (end 62.7 57.4856) (width 0.25) (layer "F.Cu") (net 1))
 (segment (start 66.7952 63.981) (end 68.426 63.981) (width 0.25) (layer "F.Cu") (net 1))
 (segment (start 57.2058 64.897) (end 57.2058 64.1046) (width 0.25) (layer "F.Cu") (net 2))
 (segment (start 62.7 62.8522) (end 62.7 61.425) (width 0.25) (layer "F.Cu") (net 2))
 (segment (start 57.912 63.3984) (end 62.1538 63.3984) (width 0.25) (layer "F.Cu") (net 2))
 (segment (start 57.2058 64.1046) (end 57.912 63.3984) (width 0.25) (layer "F.Cu") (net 2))
 (segment (start 62.1538 63.3984) (end 62.7 62.8522) (width 0.25) (layer "F.Cu") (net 2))
 (segment (start 59.4122 63.981) (end 64.5202 63.981) (width 0.25) (layer "F.Cu") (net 11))
 (segment (start 59.1058 64.2874) (end 59.4122 63.981) (width 0.25) (layer "F.Cu") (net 11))
 (segment (start 59.1058 64.897) (end 59.1058 64.2874) (width 0.25) (layer "F.Cu") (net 11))
 (segment (start 66.7952 67.346) (end 66.6602 67.481) (width 0.25) (layer "F.Cu") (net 10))
 (segment (start 67.7164 67.3608) (end 68.4276 67.3608) (width 0.25) (layer "F.Cu") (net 10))
 (segment (start 66.7952 65.881) (end 66.7952 67.196) (width 0.25) (layer "F.Cu") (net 10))
 (segment (start 66.5226 67.481) (end 67.5962 67.481) (width 0.25) (layer "F.Cu") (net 10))
 (segment (start 66.5226 67.481) (end 66.1702 67.481) (width 0.25) (layer "F.Cu") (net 10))
 (segment (start 66.7952 67.196) (end 66.7952 67.346) (width 0.25) (layer "F.Cu") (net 10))
 (segment (start 66.6602 67.481) (end 66.5226 67.481) (width 0.25) (layer "F.Cu") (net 10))
 (segment (start 67.5962 67.481) (end 67.7164 67.3608) (width 0.25) (layer "F.Cu") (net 10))
 (segment (start 59.9694 52.2478) (end 61.219 52.2478) (width 0.25) (layer "F.Cu") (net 9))
 (segment (start 59.563 52.6542) (end 59.9694 52.2478) (width 0.25) (layer "F.Cu") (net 9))
 (segment (start 64.1858 52.1208) (end 64.9438 52.1208) (width 0.25) (layer "F.Cu") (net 8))
 (segment (start 64.9732 52.0914) (end 64.9438 52.1208) (width 0.25) (layer "F.Cu") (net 8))
 (segment (start 63.3496 51.564) (end 63.3496 50.8762) (width 0.25) (layer "F.Cu") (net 8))
 (segment (start 63.494 51.7084) (end 63.3496 51.564) (width 0.25) (layer "F.Cu") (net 8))
 (segment (start 64.0588 52.2478) (end 64.1858 52.1208) (width 0.25) (layer "F.Cu") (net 8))
 (segment (start 63.494 52.2478) (end 64.0588 52.2478) (width 0.25) (layer "F.Cu") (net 8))
 (segment (start 63.494 52.2478) (end 63.494 51.7084) (width 0.25) (layer "F.Cu") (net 8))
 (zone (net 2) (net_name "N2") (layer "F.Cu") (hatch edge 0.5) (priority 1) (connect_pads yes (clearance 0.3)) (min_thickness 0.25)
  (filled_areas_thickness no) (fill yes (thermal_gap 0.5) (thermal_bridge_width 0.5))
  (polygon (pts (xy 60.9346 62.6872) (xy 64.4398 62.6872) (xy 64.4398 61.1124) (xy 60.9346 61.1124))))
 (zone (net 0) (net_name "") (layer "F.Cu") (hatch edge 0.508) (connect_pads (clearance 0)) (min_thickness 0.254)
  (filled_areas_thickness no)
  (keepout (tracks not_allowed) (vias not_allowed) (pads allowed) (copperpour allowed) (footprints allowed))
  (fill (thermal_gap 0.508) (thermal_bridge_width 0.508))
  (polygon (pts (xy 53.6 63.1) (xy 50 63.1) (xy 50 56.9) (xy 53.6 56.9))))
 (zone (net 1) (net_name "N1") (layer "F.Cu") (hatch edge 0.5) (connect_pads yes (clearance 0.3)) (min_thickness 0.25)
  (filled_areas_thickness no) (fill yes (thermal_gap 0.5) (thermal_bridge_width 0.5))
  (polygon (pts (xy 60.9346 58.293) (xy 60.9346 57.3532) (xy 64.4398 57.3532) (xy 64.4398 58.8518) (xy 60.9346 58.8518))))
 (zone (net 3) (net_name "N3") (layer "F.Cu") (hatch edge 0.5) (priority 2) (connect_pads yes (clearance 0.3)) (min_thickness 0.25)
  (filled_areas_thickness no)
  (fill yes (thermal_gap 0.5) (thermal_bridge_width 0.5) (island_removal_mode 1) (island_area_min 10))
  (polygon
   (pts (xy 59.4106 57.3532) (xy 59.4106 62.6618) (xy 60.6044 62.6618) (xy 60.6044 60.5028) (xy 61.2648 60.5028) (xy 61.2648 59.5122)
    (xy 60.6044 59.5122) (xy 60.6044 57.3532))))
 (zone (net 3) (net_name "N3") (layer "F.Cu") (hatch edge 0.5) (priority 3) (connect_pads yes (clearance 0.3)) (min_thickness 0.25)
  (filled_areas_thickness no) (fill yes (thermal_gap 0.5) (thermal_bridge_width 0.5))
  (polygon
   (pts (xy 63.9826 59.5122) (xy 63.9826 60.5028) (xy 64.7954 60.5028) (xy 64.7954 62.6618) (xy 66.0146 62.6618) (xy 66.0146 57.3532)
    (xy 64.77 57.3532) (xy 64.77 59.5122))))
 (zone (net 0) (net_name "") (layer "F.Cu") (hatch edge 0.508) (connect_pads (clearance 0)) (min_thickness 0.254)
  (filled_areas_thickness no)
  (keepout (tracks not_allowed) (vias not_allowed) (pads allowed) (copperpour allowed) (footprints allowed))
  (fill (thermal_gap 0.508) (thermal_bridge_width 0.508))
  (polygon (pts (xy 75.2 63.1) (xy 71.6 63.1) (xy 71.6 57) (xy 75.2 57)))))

